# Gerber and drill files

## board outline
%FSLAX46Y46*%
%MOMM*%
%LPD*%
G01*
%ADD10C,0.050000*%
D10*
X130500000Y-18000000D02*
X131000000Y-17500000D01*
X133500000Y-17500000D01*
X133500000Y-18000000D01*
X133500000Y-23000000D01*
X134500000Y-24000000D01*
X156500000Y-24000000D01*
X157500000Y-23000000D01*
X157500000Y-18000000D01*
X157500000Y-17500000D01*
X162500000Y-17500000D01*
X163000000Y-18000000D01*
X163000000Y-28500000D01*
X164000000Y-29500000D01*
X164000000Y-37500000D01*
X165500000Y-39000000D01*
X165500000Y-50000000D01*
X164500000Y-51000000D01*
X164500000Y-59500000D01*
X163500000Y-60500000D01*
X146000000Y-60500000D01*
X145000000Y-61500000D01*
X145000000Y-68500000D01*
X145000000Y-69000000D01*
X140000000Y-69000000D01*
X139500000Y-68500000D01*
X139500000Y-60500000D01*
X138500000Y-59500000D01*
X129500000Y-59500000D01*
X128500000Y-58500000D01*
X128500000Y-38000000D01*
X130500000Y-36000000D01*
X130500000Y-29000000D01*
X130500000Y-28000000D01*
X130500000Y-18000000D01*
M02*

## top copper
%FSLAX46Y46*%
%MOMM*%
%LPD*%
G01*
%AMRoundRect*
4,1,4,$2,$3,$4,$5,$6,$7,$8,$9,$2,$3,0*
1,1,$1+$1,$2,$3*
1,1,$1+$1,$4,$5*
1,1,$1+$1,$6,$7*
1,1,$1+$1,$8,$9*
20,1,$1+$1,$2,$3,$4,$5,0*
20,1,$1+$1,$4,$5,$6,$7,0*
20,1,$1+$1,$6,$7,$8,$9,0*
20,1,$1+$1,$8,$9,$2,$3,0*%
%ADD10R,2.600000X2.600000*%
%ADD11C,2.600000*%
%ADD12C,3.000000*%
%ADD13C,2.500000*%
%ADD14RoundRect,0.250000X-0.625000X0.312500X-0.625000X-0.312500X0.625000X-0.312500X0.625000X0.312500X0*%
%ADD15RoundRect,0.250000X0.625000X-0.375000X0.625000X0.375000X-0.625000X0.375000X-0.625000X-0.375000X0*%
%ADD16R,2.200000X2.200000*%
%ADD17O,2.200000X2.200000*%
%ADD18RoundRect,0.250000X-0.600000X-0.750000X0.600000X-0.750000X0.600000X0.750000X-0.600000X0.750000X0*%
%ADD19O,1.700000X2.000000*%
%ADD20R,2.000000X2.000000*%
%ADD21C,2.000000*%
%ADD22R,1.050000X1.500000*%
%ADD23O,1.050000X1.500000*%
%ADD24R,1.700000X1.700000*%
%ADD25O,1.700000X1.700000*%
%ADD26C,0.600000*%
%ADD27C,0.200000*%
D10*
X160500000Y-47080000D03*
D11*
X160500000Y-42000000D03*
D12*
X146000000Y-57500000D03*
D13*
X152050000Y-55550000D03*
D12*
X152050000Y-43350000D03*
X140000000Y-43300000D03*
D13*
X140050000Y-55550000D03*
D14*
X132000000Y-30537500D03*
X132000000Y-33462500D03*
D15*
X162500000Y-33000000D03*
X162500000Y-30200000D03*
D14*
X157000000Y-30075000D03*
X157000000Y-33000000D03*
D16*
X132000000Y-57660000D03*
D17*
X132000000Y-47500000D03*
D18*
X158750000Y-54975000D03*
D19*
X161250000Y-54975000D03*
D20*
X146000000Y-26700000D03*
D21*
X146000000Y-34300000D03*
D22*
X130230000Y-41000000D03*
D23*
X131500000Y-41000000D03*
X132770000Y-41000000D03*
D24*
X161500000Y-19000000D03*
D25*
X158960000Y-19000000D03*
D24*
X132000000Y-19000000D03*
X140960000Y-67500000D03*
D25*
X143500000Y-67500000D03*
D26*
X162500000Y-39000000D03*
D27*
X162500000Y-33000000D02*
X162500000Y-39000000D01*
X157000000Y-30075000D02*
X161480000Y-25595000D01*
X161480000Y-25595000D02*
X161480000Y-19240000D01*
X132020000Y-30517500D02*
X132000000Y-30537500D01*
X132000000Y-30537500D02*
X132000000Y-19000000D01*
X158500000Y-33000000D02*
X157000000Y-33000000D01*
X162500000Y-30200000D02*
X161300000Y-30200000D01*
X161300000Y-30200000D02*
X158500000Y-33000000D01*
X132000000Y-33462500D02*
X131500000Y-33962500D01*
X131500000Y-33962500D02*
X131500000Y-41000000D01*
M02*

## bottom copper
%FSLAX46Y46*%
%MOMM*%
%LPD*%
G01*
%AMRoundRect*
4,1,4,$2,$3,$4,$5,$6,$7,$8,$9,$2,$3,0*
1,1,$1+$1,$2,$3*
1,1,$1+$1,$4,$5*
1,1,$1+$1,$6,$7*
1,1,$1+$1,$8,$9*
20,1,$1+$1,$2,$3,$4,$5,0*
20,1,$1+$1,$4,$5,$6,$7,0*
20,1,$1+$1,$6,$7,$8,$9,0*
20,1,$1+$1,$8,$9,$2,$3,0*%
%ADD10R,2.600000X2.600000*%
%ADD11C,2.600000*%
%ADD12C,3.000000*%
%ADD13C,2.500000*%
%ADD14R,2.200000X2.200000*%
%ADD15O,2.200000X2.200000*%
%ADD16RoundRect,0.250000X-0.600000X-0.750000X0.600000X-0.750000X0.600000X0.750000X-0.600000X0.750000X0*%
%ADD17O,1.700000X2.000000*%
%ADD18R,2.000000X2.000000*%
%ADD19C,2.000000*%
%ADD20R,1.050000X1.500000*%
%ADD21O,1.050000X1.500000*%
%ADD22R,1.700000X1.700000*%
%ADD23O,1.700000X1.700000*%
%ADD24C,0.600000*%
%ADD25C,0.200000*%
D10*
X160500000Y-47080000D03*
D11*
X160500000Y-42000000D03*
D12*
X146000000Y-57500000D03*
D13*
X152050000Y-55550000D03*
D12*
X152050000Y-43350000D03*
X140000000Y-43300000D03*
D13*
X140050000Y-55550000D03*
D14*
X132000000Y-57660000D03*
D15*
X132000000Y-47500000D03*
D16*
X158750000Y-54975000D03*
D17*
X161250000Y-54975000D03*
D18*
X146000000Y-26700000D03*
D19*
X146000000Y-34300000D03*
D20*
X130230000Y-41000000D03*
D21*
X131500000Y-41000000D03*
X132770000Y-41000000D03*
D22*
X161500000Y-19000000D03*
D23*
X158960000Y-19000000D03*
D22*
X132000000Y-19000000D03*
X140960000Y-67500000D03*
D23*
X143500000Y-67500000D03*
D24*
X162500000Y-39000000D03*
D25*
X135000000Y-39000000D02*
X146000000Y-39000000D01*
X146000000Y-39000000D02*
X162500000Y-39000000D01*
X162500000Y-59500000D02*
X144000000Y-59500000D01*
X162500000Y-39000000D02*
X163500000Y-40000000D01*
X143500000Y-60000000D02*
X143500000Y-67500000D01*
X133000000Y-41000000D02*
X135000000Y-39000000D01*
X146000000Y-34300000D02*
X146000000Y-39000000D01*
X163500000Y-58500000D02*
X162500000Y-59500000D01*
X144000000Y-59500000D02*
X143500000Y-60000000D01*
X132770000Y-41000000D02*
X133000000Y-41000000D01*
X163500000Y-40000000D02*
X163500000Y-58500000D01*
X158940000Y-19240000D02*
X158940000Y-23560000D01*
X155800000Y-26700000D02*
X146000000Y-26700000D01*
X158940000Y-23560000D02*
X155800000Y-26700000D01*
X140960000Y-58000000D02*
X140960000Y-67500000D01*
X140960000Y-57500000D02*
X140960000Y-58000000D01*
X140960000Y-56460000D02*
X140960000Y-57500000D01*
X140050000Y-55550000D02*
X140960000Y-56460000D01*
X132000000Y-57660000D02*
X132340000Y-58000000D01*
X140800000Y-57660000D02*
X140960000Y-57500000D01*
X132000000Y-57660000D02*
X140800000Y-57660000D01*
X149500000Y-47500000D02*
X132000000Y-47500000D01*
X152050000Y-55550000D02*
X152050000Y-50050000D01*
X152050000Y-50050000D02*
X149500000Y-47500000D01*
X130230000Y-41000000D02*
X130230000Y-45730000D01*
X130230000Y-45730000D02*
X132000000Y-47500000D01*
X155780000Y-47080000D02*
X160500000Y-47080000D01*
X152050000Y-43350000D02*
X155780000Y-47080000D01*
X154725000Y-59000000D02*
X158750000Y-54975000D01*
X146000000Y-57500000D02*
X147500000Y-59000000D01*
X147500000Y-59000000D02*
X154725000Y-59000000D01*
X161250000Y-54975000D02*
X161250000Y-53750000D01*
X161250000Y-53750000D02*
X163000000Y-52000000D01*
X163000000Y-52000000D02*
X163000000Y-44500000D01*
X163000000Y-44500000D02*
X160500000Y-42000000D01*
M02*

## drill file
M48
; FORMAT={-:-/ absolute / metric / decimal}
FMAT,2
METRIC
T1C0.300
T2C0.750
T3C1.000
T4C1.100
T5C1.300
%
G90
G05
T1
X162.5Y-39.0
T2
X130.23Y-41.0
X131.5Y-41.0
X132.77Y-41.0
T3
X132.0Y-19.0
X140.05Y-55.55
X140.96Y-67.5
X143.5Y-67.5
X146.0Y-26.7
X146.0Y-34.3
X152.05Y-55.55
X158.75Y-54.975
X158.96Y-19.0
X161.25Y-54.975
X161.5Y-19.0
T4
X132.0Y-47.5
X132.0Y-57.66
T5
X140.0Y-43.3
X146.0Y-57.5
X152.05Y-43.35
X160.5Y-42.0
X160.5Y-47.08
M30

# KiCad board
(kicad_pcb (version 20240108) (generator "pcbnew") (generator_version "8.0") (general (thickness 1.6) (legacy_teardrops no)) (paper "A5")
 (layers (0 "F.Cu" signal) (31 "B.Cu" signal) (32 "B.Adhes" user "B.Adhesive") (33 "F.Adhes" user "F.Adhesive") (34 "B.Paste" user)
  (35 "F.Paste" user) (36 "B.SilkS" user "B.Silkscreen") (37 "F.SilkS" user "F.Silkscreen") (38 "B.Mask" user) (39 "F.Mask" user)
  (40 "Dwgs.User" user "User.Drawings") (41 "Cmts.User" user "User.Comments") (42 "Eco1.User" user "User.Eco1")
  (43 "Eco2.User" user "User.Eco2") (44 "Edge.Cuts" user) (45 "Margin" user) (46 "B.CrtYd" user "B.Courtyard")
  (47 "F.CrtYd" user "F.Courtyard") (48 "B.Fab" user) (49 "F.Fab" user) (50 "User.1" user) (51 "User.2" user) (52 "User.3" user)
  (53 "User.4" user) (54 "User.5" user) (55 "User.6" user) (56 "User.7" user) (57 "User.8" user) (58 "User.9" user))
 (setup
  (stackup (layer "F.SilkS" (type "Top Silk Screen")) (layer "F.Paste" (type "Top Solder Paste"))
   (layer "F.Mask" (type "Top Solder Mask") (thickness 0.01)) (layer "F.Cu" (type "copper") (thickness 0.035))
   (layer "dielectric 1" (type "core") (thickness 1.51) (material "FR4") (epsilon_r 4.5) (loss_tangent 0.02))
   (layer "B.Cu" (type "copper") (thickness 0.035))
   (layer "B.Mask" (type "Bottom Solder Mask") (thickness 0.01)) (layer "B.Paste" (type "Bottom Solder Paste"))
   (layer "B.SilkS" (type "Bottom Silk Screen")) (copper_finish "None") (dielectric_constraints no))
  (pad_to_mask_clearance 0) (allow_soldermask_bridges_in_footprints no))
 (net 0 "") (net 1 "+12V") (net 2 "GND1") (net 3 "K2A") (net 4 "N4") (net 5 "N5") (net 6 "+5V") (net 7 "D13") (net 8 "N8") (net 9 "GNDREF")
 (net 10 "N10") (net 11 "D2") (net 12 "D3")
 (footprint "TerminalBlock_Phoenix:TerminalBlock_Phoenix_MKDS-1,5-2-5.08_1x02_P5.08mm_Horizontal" (layer "F.Cu") (at 160.5 47.08 90)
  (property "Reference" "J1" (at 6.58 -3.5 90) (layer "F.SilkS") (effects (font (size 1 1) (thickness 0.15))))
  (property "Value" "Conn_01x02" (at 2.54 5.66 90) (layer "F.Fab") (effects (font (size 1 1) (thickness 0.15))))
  (pad "1" thru_hole rect (at 0 0 90) (size 2.6 2.6) (drill 1.3) (layers "*.Cu" "*.Mask") (remove_unused_layers no) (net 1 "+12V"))
  (pad "2" thru_hole circle (at 5.08 0 90) (size 2.6 2.6) (drill 1.3) (layers "*.Cu" "*.Mask") (remove_unused_layers no) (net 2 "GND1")))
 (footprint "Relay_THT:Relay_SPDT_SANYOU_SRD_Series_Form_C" (layer "F.Cu") (at 146 57.5 90)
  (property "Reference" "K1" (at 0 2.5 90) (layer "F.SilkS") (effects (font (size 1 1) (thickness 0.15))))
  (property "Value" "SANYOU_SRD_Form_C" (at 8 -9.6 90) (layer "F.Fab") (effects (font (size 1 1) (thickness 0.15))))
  (pad "1" thru_hole circle (at 0 0 180) (size 3 3) (drill 1.3) (layers "*.Cu" "*.Mask") (remove_unused_layers no) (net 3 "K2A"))
  (pad "2" thru_hole circle (at 1.95 6.05 180) (size 2.5 2.5) (drill 1) (layers "*.Cu" "*.Mask") (remove_unused_layers no) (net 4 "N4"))
  (pad "3" thru_hole circle (at 14.15 6.05 180) (size 3 3) (drill 1.3) (layers "*.Cu" "*.Mask") (remove_unused_layers no) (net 1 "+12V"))
  (pad "4" thru_hole circle (at 14.2 -6 180) (size 3 3) (drill 1.3) (layers "*.Cu" "*.Mask") (remove_unused_layers no) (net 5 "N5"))
  (pad "5" thru_hole circle (at 1.95 -5.95 180) (size 2.5 2.5) (drill 1) (layers "*.Cu" "*.Mask") (remove_unused_layers no) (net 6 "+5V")))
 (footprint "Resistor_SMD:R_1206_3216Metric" (layer "F.Cu") (at 132 32 -90)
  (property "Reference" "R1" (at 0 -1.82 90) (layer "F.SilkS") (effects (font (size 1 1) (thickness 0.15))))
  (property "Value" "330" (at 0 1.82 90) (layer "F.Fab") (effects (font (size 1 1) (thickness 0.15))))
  (pad "1" smd roundrect (at -1.4625 0 270) (size 1.125 1.75) (layers "F.Cu" "F.Paste" "F.Mask") (roundrect_rratio 0.222222) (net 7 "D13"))
  (pad "2" smd roundrect (at 1.4625 0 270) (size 1.125 1.75) (layers "F.Cu" "F.Paste" "F.Mask") (roundrect_rratio 0.222222) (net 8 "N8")))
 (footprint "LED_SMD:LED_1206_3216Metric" (layer "F.Cu") (at 162.5 31.6 90)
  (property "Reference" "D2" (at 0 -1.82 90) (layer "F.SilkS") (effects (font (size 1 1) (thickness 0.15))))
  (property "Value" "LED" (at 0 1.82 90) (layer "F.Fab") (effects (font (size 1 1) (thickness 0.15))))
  (pad "1" smd roundrect (at -1.4 0 90) (size 1.25 1.75) (layers "F.Cu" "F.Paste" "F.Mask") (roundrect_rratio 0.2) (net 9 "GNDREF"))
  (pad "2" smd roundrect (at 1.4 0 90) (size 1.25 1.75) (layers "F.Cu" "F.Paste" "F.Mask") (roundrect_rratio 0.2) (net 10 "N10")))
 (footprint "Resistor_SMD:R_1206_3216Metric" (layer "F.Cu") (at 157 31.5375 -90)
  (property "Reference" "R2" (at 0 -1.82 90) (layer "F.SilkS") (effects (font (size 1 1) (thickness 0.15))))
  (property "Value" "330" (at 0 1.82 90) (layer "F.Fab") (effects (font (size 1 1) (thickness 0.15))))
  (pad "1" smd roundrect (at -1.4625 0 270) (size 1.125 1.75) (layers "F.Cu" "F.Paste" "F.Mask") (roundrect_rratio 0.222222) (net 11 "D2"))
  (pad "2" smd roundrect (at 1.4625 0 270) (size 1.125 1.75) (layers "F.Cu" "F.Paste" "F.Mask") (roundrect_rratio 0.222222) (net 10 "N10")))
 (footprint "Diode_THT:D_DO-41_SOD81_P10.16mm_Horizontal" (layer "F.Cu") (at 132 57.66 90)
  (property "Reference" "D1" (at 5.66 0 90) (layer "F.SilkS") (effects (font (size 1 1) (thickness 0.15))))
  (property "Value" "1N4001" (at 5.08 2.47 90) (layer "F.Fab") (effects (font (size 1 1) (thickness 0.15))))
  (pad "1" thru_hole rect (at 0 0 90) (size 2.2 2.2) (drill 1.1) (layers "*.Cu" "*.Mask") (remove_unused_layers no) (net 6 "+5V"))
  (pad "2" thru_hole oval (at 10.16 0 90) (size 2.2 2.2) (drill 1.1) (layers "*.Cu" "*.Mask") (remove_unused_layers no) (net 4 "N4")))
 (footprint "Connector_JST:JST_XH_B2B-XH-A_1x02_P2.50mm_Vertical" (layer "F.Cu") (at 158.75 54.975)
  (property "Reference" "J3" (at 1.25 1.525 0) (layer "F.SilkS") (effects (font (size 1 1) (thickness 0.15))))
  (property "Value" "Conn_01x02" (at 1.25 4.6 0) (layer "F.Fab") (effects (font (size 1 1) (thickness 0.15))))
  (pad "1" thru_hole roundrect (at 0 0) (size 1.7 2) (drill 1) (layers "*.Cu" "*.Mask") (remove_unused_layers no)
   (roundrect_rratio 0.147059) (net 3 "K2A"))
  (pad "2" thru_hole oval (at 2.5 0) (size 1.7 2) (drill 1) (layers "*.Cu" "*.Mask") (remove_unused_layers no) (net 2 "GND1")))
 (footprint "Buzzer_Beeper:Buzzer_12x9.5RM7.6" (layer "F.Cu") (at 146 26.7 -90)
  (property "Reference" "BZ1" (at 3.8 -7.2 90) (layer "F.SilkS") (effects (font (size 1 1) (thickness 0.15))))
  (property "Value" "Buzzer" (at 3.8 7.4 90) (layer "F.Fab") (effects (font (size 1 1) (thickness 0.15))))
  (pad "1" thru_hole rect (at 0 0 270) (size 2 2) (drill 1) (layers "*.Cu" "*.Mask") (remove_unused_layers no) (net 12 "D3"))
  (pad "2" thru_hole circle (at 7.6 0 270) (size 2 2) (drill 1) (layers "*.Cu" "*.Mask") (remove_unused_layers no) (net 9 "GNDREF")))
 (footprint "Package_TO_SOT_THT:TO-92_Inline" (layer "F.Cu") (at 130.23 41)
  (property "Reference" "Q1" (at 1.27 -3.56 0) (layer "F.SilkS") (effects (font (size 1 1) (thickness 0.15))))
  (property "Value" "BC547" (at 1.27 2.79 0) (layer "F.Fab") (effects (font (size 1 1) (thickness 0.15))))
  (pad "1" thru_hole rect (at 0 0) (size 1.05 1.5) (drill 0.75) (layers "*.Cu" "*.Mask") (remove_unused_layers no) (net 4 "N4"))
  (pad "2" thru_hole oval (at 1.27 0) (size 1.05 1.5) (drill 0.75) (layers "*.Cu" "*.Mask") (remove_unused_layers no) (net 8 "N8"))
  (pad "3" thru_hole oval (at 2.54 0) (size 1.05 1.5) (drill 0.75) (layers "*.Cu" "*.Mask") (remove_unused_layers no) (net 9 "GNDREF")))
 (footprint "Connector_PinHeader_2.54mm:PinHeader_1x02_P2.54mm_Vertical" (layer "B.Cu") (at 161.5 19 90)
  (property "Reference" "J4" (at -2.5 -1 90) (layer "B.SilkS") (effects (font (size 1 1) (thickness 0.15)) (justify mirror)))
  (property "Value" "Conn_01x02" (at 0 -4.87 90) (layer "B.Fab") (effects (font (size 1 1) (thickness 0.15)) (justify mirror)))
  (pad "1" thru_hole rect (at 0 0 90) (size 1.7 1.7) (drill 1) (layers "*.Cu" "*.Mask") (remove_unused_layers no) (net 11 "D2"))
  (pad "2" thru_hole oval (at 0 -2.54 90) (size 1.7 1.7) (drill 1) (layers "*.Cu" "*.Mask") (remove_unused_layers no) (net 12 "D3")))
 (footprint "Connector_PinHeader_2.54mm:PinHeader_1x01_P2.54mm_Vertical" (layer "B.Cu") (at 132 19 180)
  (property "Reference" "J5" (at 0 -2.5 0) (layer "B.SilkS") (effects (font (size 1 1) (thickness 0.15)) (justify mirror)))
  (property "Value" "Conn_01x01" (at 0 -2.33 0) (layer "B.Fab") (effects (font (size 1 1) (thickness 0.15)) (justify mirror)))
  (pad "1" thru_hole rect (at 0 0 180) (size 1.7 1.7) (drill 1) (layers "*.Cu" "*.Mask") (remove_unused_layers no) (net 7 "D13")))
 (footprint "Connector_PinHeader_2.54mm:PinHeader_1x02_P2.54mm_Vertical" (layer "B.Cu") (at 140.96 67.5 -90)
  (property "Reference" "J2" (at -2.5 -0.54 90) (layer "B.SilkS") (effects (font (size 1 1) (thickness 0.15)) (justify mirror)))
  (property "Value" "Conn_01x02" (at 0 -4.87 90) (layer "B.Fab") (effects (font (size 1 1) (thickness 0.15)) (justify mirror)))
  (pad "1" thru_hole rect (at 0 0 270) (size 1.7 1.7) (drill 1) (layers "*.Cu" "*.Mask") (remove_unused_layers no) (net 6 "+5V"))
  (pad "2" thru_hole oval (at 0 -2.54 270) (size 1.7 1.7) (drill 1) (layers "*.Cu" "*.Mask") (remove_unused_layers no) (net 9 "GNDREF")))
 (gr_poly
  (pts (xy 130.5 18) (xy 131 17.5) (xy 133.5 17.5) (xy 133.5 18) (xy 133.5 23) (xy 134.5 24) (xy 156.5 24) (xy 157.5 23) (xy 157.5 18)
   (xy 157.5 17.5) (xy 162.5 17.5) (xy 163 18) (xy 163 28.5) (xy 164 29.5) (xy 164 37.5) (xy 165.5 39) (xy 165.5 50) (xy 164.5 51)
   (xy 164.5 59.5) (xy 163.5 60.5) (xy 146 60.5) (xy 145 61.5) (xy 145 68.5) (xy 145 69) (xy 140 69) (xy 139.5 68.5) (xy 139.5 60.5)
   (xy 138.5 59.5) (xy 129.5 59.5) (xy 128.5 58.5) (xy 128.5 38) (xy 130.5 36) (xy 130.5 29) (xy 130.5 28))
  (stroke (width 0.05) (type solid)) (fill none) (layer "Edge.Cuts"))
 (segment (start 162.5 33) (end 162.5 39) (width 0.2) (layer "F.Cu") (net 9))
 (via (at 162.5 39) (size 0.6) (drill 0.3) (layers "F.Cu" "B.Cu") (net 9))
 (segment (start 135 39) (end 146 39) (width 0.2) (layer "B.Cu") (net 9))
 (segment (start 146 39) (end 162.5 39) (width 0.2) (layer "B.Cu") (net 9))
 (segment (start 162.5 59.5) (end 144 59.5) (width 0.2) (layer "B.Cu") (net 9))
 (segment (start 162.5 39) (end 163.5 40) (width 0.2) (layer "B.Cu") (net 9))
 (segment (start 143.5 60) (end 143.5 67.5) (width 0.2) (layer "B.Cu") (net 9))
 (segment (start 133 41) (end 135 39) (width 0.2) (layer "B.Cu") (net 9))
 (segment (start 146 34.3) (end 146 39) (width 0.2) (layer "B.Cu") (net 9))
 (segment (start 163.5 58.5) (end 162.5 59.5) (width 0.2) (layer "B.Cu") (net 9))
 (segment (start 144 59.5) (end 143.5 60) (width 0.2) (layer "B.Cu") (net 9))
 (segment (start 132.77 41) (end 133 41) (width 0.2) (layer "B.Cu") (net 9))
 (segment (start 163.5 40) (end 163.5 58.5) (width 0.2) (layer "B.Cu") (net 9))
 (segment (start 157 30.075) (end 161.48 25.595) (width 0.2) (layer "F.Cu") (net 11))
 (segment (start 161.48 25.595) (end 161.48 19.24) (width 0.2) (layer "F.Cu") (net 11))
 (segment (start 132.02 30.5175) (end 132 30.5375) (width 0.2) (layer "F.Cu") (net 7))
 (segment (start 132 30.5375) (end 132 19) (width 0.2) (layer "F.Cu") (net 7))
 (segment (start 158.94 19.24) (end 158.94 23.56) (width 0.2) (layer "B.Cu") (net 12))
 (segment (start 155.8 26.7) (end 146 26.7) (width 0.2) (layer "B.Cu") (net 12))
 (segment (start 158.94 23.56) (end 155.8 26.7) (width 0.2) (layer "B.Cu") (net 12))
 (segment (start 140.96 58) (end 140.96 67.5) (width 0.2) (layer "B.Cu") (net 6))
 (segment (start 140.96 57.5) (end 140.96 58) (width 0.2) (layer "B.Cu") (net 6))
 (segment (start 140.96 56.46) (end 140.96 57.5) (width 0.2) (layer "B.Cu") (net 6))
 (segment (start 140.05 55.55) (end 140.96 56.46) (width 0.2) (layer "B.Cu") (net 6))
 (segment (start 132 57.66) (end 132.34 58) (width 0.2) (layer "B.Cu") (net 6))
 (segment (start 140.8 57.66) (end 140.96 57.5) (width 0.2) (layer "B.Cu") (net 6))
 (segment (start 132 57.66) (end 140.8 57.66) (width 0.2) (layer "B.Cu") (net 6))
 (segment (start 149.5 47.5) (end 132 47.5) (width 0.2) (layer "B.Cu") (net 4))
 (segment (start 152.05 55.55) (end 152.05 50.05) (width 0.2) (layer "B.Cu") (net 4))
 (segment (start 152.05 50.05) (end 149.5 47.5) (width 0.2) (layer "B.Cu") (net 4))
 (segment (start 130.23 41) (end 130.23 45.73) (width 0.2) (layer "B.Cu") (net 4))
 (segment (start 130.23 45.73) (end 132 47.5) (width 0.2) (layer "B.Cu") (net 4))
 (segment (start 158.5 33) (end 157 33) (width 0.2) (layer "F.Cu") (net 10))
 (segment (start 162.5 30.2) (end 161.3 30.2) (width 0.2) (layer "F.Cu") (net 10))
 (segment (start 161.3 30.2) (end 158.5 33) (width 0.2) (layer "F.Cu") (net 10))
 (segment (start 155.78 47.08) (end 160.5 47.08) (width 0.2) (layer "B.Cu") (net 1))
 (segment (start 152.05 43.35) (end 155.78 47.08) (width 0.2) (layer "B.Cu") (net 1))
 (segment (start 154.725 59) (end 158.75 54.975) (width 0.2) (layer "B.Cu") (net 3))
 (segment (start 146 57.5) (end 147.5 59) (width 0.2) (layer "B.Cu") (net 3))
 (segment (start 147.5 59) (end 154.725 59) (width 0.2) (layer "B.Cu") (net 3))
 (segment (start 132 33.4625) (end 131.5 33.9625) (width 0.2) (layer "F.Cu") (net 8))
 (segment (start 131.5 33.9625) (end 131.5 41) (width 0.2) (layer "F.Cu") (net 8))
 (segment (start 161.25 54.975) (end 161.25 53.75) (width 0.2) (layer "B.Cu") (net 2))
 (segment (start 161.25 53.75) (end 163 52) (width 0.2) (layer "B.Cu") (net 2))
 (segment (start 163 52) (end 163 44.5) (width 0.2) (layer "B.Cu") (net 2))
 (segment (start 163 44.5) (end 160.5 42) (width 0.2) (layer "B.Cu") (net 2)))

